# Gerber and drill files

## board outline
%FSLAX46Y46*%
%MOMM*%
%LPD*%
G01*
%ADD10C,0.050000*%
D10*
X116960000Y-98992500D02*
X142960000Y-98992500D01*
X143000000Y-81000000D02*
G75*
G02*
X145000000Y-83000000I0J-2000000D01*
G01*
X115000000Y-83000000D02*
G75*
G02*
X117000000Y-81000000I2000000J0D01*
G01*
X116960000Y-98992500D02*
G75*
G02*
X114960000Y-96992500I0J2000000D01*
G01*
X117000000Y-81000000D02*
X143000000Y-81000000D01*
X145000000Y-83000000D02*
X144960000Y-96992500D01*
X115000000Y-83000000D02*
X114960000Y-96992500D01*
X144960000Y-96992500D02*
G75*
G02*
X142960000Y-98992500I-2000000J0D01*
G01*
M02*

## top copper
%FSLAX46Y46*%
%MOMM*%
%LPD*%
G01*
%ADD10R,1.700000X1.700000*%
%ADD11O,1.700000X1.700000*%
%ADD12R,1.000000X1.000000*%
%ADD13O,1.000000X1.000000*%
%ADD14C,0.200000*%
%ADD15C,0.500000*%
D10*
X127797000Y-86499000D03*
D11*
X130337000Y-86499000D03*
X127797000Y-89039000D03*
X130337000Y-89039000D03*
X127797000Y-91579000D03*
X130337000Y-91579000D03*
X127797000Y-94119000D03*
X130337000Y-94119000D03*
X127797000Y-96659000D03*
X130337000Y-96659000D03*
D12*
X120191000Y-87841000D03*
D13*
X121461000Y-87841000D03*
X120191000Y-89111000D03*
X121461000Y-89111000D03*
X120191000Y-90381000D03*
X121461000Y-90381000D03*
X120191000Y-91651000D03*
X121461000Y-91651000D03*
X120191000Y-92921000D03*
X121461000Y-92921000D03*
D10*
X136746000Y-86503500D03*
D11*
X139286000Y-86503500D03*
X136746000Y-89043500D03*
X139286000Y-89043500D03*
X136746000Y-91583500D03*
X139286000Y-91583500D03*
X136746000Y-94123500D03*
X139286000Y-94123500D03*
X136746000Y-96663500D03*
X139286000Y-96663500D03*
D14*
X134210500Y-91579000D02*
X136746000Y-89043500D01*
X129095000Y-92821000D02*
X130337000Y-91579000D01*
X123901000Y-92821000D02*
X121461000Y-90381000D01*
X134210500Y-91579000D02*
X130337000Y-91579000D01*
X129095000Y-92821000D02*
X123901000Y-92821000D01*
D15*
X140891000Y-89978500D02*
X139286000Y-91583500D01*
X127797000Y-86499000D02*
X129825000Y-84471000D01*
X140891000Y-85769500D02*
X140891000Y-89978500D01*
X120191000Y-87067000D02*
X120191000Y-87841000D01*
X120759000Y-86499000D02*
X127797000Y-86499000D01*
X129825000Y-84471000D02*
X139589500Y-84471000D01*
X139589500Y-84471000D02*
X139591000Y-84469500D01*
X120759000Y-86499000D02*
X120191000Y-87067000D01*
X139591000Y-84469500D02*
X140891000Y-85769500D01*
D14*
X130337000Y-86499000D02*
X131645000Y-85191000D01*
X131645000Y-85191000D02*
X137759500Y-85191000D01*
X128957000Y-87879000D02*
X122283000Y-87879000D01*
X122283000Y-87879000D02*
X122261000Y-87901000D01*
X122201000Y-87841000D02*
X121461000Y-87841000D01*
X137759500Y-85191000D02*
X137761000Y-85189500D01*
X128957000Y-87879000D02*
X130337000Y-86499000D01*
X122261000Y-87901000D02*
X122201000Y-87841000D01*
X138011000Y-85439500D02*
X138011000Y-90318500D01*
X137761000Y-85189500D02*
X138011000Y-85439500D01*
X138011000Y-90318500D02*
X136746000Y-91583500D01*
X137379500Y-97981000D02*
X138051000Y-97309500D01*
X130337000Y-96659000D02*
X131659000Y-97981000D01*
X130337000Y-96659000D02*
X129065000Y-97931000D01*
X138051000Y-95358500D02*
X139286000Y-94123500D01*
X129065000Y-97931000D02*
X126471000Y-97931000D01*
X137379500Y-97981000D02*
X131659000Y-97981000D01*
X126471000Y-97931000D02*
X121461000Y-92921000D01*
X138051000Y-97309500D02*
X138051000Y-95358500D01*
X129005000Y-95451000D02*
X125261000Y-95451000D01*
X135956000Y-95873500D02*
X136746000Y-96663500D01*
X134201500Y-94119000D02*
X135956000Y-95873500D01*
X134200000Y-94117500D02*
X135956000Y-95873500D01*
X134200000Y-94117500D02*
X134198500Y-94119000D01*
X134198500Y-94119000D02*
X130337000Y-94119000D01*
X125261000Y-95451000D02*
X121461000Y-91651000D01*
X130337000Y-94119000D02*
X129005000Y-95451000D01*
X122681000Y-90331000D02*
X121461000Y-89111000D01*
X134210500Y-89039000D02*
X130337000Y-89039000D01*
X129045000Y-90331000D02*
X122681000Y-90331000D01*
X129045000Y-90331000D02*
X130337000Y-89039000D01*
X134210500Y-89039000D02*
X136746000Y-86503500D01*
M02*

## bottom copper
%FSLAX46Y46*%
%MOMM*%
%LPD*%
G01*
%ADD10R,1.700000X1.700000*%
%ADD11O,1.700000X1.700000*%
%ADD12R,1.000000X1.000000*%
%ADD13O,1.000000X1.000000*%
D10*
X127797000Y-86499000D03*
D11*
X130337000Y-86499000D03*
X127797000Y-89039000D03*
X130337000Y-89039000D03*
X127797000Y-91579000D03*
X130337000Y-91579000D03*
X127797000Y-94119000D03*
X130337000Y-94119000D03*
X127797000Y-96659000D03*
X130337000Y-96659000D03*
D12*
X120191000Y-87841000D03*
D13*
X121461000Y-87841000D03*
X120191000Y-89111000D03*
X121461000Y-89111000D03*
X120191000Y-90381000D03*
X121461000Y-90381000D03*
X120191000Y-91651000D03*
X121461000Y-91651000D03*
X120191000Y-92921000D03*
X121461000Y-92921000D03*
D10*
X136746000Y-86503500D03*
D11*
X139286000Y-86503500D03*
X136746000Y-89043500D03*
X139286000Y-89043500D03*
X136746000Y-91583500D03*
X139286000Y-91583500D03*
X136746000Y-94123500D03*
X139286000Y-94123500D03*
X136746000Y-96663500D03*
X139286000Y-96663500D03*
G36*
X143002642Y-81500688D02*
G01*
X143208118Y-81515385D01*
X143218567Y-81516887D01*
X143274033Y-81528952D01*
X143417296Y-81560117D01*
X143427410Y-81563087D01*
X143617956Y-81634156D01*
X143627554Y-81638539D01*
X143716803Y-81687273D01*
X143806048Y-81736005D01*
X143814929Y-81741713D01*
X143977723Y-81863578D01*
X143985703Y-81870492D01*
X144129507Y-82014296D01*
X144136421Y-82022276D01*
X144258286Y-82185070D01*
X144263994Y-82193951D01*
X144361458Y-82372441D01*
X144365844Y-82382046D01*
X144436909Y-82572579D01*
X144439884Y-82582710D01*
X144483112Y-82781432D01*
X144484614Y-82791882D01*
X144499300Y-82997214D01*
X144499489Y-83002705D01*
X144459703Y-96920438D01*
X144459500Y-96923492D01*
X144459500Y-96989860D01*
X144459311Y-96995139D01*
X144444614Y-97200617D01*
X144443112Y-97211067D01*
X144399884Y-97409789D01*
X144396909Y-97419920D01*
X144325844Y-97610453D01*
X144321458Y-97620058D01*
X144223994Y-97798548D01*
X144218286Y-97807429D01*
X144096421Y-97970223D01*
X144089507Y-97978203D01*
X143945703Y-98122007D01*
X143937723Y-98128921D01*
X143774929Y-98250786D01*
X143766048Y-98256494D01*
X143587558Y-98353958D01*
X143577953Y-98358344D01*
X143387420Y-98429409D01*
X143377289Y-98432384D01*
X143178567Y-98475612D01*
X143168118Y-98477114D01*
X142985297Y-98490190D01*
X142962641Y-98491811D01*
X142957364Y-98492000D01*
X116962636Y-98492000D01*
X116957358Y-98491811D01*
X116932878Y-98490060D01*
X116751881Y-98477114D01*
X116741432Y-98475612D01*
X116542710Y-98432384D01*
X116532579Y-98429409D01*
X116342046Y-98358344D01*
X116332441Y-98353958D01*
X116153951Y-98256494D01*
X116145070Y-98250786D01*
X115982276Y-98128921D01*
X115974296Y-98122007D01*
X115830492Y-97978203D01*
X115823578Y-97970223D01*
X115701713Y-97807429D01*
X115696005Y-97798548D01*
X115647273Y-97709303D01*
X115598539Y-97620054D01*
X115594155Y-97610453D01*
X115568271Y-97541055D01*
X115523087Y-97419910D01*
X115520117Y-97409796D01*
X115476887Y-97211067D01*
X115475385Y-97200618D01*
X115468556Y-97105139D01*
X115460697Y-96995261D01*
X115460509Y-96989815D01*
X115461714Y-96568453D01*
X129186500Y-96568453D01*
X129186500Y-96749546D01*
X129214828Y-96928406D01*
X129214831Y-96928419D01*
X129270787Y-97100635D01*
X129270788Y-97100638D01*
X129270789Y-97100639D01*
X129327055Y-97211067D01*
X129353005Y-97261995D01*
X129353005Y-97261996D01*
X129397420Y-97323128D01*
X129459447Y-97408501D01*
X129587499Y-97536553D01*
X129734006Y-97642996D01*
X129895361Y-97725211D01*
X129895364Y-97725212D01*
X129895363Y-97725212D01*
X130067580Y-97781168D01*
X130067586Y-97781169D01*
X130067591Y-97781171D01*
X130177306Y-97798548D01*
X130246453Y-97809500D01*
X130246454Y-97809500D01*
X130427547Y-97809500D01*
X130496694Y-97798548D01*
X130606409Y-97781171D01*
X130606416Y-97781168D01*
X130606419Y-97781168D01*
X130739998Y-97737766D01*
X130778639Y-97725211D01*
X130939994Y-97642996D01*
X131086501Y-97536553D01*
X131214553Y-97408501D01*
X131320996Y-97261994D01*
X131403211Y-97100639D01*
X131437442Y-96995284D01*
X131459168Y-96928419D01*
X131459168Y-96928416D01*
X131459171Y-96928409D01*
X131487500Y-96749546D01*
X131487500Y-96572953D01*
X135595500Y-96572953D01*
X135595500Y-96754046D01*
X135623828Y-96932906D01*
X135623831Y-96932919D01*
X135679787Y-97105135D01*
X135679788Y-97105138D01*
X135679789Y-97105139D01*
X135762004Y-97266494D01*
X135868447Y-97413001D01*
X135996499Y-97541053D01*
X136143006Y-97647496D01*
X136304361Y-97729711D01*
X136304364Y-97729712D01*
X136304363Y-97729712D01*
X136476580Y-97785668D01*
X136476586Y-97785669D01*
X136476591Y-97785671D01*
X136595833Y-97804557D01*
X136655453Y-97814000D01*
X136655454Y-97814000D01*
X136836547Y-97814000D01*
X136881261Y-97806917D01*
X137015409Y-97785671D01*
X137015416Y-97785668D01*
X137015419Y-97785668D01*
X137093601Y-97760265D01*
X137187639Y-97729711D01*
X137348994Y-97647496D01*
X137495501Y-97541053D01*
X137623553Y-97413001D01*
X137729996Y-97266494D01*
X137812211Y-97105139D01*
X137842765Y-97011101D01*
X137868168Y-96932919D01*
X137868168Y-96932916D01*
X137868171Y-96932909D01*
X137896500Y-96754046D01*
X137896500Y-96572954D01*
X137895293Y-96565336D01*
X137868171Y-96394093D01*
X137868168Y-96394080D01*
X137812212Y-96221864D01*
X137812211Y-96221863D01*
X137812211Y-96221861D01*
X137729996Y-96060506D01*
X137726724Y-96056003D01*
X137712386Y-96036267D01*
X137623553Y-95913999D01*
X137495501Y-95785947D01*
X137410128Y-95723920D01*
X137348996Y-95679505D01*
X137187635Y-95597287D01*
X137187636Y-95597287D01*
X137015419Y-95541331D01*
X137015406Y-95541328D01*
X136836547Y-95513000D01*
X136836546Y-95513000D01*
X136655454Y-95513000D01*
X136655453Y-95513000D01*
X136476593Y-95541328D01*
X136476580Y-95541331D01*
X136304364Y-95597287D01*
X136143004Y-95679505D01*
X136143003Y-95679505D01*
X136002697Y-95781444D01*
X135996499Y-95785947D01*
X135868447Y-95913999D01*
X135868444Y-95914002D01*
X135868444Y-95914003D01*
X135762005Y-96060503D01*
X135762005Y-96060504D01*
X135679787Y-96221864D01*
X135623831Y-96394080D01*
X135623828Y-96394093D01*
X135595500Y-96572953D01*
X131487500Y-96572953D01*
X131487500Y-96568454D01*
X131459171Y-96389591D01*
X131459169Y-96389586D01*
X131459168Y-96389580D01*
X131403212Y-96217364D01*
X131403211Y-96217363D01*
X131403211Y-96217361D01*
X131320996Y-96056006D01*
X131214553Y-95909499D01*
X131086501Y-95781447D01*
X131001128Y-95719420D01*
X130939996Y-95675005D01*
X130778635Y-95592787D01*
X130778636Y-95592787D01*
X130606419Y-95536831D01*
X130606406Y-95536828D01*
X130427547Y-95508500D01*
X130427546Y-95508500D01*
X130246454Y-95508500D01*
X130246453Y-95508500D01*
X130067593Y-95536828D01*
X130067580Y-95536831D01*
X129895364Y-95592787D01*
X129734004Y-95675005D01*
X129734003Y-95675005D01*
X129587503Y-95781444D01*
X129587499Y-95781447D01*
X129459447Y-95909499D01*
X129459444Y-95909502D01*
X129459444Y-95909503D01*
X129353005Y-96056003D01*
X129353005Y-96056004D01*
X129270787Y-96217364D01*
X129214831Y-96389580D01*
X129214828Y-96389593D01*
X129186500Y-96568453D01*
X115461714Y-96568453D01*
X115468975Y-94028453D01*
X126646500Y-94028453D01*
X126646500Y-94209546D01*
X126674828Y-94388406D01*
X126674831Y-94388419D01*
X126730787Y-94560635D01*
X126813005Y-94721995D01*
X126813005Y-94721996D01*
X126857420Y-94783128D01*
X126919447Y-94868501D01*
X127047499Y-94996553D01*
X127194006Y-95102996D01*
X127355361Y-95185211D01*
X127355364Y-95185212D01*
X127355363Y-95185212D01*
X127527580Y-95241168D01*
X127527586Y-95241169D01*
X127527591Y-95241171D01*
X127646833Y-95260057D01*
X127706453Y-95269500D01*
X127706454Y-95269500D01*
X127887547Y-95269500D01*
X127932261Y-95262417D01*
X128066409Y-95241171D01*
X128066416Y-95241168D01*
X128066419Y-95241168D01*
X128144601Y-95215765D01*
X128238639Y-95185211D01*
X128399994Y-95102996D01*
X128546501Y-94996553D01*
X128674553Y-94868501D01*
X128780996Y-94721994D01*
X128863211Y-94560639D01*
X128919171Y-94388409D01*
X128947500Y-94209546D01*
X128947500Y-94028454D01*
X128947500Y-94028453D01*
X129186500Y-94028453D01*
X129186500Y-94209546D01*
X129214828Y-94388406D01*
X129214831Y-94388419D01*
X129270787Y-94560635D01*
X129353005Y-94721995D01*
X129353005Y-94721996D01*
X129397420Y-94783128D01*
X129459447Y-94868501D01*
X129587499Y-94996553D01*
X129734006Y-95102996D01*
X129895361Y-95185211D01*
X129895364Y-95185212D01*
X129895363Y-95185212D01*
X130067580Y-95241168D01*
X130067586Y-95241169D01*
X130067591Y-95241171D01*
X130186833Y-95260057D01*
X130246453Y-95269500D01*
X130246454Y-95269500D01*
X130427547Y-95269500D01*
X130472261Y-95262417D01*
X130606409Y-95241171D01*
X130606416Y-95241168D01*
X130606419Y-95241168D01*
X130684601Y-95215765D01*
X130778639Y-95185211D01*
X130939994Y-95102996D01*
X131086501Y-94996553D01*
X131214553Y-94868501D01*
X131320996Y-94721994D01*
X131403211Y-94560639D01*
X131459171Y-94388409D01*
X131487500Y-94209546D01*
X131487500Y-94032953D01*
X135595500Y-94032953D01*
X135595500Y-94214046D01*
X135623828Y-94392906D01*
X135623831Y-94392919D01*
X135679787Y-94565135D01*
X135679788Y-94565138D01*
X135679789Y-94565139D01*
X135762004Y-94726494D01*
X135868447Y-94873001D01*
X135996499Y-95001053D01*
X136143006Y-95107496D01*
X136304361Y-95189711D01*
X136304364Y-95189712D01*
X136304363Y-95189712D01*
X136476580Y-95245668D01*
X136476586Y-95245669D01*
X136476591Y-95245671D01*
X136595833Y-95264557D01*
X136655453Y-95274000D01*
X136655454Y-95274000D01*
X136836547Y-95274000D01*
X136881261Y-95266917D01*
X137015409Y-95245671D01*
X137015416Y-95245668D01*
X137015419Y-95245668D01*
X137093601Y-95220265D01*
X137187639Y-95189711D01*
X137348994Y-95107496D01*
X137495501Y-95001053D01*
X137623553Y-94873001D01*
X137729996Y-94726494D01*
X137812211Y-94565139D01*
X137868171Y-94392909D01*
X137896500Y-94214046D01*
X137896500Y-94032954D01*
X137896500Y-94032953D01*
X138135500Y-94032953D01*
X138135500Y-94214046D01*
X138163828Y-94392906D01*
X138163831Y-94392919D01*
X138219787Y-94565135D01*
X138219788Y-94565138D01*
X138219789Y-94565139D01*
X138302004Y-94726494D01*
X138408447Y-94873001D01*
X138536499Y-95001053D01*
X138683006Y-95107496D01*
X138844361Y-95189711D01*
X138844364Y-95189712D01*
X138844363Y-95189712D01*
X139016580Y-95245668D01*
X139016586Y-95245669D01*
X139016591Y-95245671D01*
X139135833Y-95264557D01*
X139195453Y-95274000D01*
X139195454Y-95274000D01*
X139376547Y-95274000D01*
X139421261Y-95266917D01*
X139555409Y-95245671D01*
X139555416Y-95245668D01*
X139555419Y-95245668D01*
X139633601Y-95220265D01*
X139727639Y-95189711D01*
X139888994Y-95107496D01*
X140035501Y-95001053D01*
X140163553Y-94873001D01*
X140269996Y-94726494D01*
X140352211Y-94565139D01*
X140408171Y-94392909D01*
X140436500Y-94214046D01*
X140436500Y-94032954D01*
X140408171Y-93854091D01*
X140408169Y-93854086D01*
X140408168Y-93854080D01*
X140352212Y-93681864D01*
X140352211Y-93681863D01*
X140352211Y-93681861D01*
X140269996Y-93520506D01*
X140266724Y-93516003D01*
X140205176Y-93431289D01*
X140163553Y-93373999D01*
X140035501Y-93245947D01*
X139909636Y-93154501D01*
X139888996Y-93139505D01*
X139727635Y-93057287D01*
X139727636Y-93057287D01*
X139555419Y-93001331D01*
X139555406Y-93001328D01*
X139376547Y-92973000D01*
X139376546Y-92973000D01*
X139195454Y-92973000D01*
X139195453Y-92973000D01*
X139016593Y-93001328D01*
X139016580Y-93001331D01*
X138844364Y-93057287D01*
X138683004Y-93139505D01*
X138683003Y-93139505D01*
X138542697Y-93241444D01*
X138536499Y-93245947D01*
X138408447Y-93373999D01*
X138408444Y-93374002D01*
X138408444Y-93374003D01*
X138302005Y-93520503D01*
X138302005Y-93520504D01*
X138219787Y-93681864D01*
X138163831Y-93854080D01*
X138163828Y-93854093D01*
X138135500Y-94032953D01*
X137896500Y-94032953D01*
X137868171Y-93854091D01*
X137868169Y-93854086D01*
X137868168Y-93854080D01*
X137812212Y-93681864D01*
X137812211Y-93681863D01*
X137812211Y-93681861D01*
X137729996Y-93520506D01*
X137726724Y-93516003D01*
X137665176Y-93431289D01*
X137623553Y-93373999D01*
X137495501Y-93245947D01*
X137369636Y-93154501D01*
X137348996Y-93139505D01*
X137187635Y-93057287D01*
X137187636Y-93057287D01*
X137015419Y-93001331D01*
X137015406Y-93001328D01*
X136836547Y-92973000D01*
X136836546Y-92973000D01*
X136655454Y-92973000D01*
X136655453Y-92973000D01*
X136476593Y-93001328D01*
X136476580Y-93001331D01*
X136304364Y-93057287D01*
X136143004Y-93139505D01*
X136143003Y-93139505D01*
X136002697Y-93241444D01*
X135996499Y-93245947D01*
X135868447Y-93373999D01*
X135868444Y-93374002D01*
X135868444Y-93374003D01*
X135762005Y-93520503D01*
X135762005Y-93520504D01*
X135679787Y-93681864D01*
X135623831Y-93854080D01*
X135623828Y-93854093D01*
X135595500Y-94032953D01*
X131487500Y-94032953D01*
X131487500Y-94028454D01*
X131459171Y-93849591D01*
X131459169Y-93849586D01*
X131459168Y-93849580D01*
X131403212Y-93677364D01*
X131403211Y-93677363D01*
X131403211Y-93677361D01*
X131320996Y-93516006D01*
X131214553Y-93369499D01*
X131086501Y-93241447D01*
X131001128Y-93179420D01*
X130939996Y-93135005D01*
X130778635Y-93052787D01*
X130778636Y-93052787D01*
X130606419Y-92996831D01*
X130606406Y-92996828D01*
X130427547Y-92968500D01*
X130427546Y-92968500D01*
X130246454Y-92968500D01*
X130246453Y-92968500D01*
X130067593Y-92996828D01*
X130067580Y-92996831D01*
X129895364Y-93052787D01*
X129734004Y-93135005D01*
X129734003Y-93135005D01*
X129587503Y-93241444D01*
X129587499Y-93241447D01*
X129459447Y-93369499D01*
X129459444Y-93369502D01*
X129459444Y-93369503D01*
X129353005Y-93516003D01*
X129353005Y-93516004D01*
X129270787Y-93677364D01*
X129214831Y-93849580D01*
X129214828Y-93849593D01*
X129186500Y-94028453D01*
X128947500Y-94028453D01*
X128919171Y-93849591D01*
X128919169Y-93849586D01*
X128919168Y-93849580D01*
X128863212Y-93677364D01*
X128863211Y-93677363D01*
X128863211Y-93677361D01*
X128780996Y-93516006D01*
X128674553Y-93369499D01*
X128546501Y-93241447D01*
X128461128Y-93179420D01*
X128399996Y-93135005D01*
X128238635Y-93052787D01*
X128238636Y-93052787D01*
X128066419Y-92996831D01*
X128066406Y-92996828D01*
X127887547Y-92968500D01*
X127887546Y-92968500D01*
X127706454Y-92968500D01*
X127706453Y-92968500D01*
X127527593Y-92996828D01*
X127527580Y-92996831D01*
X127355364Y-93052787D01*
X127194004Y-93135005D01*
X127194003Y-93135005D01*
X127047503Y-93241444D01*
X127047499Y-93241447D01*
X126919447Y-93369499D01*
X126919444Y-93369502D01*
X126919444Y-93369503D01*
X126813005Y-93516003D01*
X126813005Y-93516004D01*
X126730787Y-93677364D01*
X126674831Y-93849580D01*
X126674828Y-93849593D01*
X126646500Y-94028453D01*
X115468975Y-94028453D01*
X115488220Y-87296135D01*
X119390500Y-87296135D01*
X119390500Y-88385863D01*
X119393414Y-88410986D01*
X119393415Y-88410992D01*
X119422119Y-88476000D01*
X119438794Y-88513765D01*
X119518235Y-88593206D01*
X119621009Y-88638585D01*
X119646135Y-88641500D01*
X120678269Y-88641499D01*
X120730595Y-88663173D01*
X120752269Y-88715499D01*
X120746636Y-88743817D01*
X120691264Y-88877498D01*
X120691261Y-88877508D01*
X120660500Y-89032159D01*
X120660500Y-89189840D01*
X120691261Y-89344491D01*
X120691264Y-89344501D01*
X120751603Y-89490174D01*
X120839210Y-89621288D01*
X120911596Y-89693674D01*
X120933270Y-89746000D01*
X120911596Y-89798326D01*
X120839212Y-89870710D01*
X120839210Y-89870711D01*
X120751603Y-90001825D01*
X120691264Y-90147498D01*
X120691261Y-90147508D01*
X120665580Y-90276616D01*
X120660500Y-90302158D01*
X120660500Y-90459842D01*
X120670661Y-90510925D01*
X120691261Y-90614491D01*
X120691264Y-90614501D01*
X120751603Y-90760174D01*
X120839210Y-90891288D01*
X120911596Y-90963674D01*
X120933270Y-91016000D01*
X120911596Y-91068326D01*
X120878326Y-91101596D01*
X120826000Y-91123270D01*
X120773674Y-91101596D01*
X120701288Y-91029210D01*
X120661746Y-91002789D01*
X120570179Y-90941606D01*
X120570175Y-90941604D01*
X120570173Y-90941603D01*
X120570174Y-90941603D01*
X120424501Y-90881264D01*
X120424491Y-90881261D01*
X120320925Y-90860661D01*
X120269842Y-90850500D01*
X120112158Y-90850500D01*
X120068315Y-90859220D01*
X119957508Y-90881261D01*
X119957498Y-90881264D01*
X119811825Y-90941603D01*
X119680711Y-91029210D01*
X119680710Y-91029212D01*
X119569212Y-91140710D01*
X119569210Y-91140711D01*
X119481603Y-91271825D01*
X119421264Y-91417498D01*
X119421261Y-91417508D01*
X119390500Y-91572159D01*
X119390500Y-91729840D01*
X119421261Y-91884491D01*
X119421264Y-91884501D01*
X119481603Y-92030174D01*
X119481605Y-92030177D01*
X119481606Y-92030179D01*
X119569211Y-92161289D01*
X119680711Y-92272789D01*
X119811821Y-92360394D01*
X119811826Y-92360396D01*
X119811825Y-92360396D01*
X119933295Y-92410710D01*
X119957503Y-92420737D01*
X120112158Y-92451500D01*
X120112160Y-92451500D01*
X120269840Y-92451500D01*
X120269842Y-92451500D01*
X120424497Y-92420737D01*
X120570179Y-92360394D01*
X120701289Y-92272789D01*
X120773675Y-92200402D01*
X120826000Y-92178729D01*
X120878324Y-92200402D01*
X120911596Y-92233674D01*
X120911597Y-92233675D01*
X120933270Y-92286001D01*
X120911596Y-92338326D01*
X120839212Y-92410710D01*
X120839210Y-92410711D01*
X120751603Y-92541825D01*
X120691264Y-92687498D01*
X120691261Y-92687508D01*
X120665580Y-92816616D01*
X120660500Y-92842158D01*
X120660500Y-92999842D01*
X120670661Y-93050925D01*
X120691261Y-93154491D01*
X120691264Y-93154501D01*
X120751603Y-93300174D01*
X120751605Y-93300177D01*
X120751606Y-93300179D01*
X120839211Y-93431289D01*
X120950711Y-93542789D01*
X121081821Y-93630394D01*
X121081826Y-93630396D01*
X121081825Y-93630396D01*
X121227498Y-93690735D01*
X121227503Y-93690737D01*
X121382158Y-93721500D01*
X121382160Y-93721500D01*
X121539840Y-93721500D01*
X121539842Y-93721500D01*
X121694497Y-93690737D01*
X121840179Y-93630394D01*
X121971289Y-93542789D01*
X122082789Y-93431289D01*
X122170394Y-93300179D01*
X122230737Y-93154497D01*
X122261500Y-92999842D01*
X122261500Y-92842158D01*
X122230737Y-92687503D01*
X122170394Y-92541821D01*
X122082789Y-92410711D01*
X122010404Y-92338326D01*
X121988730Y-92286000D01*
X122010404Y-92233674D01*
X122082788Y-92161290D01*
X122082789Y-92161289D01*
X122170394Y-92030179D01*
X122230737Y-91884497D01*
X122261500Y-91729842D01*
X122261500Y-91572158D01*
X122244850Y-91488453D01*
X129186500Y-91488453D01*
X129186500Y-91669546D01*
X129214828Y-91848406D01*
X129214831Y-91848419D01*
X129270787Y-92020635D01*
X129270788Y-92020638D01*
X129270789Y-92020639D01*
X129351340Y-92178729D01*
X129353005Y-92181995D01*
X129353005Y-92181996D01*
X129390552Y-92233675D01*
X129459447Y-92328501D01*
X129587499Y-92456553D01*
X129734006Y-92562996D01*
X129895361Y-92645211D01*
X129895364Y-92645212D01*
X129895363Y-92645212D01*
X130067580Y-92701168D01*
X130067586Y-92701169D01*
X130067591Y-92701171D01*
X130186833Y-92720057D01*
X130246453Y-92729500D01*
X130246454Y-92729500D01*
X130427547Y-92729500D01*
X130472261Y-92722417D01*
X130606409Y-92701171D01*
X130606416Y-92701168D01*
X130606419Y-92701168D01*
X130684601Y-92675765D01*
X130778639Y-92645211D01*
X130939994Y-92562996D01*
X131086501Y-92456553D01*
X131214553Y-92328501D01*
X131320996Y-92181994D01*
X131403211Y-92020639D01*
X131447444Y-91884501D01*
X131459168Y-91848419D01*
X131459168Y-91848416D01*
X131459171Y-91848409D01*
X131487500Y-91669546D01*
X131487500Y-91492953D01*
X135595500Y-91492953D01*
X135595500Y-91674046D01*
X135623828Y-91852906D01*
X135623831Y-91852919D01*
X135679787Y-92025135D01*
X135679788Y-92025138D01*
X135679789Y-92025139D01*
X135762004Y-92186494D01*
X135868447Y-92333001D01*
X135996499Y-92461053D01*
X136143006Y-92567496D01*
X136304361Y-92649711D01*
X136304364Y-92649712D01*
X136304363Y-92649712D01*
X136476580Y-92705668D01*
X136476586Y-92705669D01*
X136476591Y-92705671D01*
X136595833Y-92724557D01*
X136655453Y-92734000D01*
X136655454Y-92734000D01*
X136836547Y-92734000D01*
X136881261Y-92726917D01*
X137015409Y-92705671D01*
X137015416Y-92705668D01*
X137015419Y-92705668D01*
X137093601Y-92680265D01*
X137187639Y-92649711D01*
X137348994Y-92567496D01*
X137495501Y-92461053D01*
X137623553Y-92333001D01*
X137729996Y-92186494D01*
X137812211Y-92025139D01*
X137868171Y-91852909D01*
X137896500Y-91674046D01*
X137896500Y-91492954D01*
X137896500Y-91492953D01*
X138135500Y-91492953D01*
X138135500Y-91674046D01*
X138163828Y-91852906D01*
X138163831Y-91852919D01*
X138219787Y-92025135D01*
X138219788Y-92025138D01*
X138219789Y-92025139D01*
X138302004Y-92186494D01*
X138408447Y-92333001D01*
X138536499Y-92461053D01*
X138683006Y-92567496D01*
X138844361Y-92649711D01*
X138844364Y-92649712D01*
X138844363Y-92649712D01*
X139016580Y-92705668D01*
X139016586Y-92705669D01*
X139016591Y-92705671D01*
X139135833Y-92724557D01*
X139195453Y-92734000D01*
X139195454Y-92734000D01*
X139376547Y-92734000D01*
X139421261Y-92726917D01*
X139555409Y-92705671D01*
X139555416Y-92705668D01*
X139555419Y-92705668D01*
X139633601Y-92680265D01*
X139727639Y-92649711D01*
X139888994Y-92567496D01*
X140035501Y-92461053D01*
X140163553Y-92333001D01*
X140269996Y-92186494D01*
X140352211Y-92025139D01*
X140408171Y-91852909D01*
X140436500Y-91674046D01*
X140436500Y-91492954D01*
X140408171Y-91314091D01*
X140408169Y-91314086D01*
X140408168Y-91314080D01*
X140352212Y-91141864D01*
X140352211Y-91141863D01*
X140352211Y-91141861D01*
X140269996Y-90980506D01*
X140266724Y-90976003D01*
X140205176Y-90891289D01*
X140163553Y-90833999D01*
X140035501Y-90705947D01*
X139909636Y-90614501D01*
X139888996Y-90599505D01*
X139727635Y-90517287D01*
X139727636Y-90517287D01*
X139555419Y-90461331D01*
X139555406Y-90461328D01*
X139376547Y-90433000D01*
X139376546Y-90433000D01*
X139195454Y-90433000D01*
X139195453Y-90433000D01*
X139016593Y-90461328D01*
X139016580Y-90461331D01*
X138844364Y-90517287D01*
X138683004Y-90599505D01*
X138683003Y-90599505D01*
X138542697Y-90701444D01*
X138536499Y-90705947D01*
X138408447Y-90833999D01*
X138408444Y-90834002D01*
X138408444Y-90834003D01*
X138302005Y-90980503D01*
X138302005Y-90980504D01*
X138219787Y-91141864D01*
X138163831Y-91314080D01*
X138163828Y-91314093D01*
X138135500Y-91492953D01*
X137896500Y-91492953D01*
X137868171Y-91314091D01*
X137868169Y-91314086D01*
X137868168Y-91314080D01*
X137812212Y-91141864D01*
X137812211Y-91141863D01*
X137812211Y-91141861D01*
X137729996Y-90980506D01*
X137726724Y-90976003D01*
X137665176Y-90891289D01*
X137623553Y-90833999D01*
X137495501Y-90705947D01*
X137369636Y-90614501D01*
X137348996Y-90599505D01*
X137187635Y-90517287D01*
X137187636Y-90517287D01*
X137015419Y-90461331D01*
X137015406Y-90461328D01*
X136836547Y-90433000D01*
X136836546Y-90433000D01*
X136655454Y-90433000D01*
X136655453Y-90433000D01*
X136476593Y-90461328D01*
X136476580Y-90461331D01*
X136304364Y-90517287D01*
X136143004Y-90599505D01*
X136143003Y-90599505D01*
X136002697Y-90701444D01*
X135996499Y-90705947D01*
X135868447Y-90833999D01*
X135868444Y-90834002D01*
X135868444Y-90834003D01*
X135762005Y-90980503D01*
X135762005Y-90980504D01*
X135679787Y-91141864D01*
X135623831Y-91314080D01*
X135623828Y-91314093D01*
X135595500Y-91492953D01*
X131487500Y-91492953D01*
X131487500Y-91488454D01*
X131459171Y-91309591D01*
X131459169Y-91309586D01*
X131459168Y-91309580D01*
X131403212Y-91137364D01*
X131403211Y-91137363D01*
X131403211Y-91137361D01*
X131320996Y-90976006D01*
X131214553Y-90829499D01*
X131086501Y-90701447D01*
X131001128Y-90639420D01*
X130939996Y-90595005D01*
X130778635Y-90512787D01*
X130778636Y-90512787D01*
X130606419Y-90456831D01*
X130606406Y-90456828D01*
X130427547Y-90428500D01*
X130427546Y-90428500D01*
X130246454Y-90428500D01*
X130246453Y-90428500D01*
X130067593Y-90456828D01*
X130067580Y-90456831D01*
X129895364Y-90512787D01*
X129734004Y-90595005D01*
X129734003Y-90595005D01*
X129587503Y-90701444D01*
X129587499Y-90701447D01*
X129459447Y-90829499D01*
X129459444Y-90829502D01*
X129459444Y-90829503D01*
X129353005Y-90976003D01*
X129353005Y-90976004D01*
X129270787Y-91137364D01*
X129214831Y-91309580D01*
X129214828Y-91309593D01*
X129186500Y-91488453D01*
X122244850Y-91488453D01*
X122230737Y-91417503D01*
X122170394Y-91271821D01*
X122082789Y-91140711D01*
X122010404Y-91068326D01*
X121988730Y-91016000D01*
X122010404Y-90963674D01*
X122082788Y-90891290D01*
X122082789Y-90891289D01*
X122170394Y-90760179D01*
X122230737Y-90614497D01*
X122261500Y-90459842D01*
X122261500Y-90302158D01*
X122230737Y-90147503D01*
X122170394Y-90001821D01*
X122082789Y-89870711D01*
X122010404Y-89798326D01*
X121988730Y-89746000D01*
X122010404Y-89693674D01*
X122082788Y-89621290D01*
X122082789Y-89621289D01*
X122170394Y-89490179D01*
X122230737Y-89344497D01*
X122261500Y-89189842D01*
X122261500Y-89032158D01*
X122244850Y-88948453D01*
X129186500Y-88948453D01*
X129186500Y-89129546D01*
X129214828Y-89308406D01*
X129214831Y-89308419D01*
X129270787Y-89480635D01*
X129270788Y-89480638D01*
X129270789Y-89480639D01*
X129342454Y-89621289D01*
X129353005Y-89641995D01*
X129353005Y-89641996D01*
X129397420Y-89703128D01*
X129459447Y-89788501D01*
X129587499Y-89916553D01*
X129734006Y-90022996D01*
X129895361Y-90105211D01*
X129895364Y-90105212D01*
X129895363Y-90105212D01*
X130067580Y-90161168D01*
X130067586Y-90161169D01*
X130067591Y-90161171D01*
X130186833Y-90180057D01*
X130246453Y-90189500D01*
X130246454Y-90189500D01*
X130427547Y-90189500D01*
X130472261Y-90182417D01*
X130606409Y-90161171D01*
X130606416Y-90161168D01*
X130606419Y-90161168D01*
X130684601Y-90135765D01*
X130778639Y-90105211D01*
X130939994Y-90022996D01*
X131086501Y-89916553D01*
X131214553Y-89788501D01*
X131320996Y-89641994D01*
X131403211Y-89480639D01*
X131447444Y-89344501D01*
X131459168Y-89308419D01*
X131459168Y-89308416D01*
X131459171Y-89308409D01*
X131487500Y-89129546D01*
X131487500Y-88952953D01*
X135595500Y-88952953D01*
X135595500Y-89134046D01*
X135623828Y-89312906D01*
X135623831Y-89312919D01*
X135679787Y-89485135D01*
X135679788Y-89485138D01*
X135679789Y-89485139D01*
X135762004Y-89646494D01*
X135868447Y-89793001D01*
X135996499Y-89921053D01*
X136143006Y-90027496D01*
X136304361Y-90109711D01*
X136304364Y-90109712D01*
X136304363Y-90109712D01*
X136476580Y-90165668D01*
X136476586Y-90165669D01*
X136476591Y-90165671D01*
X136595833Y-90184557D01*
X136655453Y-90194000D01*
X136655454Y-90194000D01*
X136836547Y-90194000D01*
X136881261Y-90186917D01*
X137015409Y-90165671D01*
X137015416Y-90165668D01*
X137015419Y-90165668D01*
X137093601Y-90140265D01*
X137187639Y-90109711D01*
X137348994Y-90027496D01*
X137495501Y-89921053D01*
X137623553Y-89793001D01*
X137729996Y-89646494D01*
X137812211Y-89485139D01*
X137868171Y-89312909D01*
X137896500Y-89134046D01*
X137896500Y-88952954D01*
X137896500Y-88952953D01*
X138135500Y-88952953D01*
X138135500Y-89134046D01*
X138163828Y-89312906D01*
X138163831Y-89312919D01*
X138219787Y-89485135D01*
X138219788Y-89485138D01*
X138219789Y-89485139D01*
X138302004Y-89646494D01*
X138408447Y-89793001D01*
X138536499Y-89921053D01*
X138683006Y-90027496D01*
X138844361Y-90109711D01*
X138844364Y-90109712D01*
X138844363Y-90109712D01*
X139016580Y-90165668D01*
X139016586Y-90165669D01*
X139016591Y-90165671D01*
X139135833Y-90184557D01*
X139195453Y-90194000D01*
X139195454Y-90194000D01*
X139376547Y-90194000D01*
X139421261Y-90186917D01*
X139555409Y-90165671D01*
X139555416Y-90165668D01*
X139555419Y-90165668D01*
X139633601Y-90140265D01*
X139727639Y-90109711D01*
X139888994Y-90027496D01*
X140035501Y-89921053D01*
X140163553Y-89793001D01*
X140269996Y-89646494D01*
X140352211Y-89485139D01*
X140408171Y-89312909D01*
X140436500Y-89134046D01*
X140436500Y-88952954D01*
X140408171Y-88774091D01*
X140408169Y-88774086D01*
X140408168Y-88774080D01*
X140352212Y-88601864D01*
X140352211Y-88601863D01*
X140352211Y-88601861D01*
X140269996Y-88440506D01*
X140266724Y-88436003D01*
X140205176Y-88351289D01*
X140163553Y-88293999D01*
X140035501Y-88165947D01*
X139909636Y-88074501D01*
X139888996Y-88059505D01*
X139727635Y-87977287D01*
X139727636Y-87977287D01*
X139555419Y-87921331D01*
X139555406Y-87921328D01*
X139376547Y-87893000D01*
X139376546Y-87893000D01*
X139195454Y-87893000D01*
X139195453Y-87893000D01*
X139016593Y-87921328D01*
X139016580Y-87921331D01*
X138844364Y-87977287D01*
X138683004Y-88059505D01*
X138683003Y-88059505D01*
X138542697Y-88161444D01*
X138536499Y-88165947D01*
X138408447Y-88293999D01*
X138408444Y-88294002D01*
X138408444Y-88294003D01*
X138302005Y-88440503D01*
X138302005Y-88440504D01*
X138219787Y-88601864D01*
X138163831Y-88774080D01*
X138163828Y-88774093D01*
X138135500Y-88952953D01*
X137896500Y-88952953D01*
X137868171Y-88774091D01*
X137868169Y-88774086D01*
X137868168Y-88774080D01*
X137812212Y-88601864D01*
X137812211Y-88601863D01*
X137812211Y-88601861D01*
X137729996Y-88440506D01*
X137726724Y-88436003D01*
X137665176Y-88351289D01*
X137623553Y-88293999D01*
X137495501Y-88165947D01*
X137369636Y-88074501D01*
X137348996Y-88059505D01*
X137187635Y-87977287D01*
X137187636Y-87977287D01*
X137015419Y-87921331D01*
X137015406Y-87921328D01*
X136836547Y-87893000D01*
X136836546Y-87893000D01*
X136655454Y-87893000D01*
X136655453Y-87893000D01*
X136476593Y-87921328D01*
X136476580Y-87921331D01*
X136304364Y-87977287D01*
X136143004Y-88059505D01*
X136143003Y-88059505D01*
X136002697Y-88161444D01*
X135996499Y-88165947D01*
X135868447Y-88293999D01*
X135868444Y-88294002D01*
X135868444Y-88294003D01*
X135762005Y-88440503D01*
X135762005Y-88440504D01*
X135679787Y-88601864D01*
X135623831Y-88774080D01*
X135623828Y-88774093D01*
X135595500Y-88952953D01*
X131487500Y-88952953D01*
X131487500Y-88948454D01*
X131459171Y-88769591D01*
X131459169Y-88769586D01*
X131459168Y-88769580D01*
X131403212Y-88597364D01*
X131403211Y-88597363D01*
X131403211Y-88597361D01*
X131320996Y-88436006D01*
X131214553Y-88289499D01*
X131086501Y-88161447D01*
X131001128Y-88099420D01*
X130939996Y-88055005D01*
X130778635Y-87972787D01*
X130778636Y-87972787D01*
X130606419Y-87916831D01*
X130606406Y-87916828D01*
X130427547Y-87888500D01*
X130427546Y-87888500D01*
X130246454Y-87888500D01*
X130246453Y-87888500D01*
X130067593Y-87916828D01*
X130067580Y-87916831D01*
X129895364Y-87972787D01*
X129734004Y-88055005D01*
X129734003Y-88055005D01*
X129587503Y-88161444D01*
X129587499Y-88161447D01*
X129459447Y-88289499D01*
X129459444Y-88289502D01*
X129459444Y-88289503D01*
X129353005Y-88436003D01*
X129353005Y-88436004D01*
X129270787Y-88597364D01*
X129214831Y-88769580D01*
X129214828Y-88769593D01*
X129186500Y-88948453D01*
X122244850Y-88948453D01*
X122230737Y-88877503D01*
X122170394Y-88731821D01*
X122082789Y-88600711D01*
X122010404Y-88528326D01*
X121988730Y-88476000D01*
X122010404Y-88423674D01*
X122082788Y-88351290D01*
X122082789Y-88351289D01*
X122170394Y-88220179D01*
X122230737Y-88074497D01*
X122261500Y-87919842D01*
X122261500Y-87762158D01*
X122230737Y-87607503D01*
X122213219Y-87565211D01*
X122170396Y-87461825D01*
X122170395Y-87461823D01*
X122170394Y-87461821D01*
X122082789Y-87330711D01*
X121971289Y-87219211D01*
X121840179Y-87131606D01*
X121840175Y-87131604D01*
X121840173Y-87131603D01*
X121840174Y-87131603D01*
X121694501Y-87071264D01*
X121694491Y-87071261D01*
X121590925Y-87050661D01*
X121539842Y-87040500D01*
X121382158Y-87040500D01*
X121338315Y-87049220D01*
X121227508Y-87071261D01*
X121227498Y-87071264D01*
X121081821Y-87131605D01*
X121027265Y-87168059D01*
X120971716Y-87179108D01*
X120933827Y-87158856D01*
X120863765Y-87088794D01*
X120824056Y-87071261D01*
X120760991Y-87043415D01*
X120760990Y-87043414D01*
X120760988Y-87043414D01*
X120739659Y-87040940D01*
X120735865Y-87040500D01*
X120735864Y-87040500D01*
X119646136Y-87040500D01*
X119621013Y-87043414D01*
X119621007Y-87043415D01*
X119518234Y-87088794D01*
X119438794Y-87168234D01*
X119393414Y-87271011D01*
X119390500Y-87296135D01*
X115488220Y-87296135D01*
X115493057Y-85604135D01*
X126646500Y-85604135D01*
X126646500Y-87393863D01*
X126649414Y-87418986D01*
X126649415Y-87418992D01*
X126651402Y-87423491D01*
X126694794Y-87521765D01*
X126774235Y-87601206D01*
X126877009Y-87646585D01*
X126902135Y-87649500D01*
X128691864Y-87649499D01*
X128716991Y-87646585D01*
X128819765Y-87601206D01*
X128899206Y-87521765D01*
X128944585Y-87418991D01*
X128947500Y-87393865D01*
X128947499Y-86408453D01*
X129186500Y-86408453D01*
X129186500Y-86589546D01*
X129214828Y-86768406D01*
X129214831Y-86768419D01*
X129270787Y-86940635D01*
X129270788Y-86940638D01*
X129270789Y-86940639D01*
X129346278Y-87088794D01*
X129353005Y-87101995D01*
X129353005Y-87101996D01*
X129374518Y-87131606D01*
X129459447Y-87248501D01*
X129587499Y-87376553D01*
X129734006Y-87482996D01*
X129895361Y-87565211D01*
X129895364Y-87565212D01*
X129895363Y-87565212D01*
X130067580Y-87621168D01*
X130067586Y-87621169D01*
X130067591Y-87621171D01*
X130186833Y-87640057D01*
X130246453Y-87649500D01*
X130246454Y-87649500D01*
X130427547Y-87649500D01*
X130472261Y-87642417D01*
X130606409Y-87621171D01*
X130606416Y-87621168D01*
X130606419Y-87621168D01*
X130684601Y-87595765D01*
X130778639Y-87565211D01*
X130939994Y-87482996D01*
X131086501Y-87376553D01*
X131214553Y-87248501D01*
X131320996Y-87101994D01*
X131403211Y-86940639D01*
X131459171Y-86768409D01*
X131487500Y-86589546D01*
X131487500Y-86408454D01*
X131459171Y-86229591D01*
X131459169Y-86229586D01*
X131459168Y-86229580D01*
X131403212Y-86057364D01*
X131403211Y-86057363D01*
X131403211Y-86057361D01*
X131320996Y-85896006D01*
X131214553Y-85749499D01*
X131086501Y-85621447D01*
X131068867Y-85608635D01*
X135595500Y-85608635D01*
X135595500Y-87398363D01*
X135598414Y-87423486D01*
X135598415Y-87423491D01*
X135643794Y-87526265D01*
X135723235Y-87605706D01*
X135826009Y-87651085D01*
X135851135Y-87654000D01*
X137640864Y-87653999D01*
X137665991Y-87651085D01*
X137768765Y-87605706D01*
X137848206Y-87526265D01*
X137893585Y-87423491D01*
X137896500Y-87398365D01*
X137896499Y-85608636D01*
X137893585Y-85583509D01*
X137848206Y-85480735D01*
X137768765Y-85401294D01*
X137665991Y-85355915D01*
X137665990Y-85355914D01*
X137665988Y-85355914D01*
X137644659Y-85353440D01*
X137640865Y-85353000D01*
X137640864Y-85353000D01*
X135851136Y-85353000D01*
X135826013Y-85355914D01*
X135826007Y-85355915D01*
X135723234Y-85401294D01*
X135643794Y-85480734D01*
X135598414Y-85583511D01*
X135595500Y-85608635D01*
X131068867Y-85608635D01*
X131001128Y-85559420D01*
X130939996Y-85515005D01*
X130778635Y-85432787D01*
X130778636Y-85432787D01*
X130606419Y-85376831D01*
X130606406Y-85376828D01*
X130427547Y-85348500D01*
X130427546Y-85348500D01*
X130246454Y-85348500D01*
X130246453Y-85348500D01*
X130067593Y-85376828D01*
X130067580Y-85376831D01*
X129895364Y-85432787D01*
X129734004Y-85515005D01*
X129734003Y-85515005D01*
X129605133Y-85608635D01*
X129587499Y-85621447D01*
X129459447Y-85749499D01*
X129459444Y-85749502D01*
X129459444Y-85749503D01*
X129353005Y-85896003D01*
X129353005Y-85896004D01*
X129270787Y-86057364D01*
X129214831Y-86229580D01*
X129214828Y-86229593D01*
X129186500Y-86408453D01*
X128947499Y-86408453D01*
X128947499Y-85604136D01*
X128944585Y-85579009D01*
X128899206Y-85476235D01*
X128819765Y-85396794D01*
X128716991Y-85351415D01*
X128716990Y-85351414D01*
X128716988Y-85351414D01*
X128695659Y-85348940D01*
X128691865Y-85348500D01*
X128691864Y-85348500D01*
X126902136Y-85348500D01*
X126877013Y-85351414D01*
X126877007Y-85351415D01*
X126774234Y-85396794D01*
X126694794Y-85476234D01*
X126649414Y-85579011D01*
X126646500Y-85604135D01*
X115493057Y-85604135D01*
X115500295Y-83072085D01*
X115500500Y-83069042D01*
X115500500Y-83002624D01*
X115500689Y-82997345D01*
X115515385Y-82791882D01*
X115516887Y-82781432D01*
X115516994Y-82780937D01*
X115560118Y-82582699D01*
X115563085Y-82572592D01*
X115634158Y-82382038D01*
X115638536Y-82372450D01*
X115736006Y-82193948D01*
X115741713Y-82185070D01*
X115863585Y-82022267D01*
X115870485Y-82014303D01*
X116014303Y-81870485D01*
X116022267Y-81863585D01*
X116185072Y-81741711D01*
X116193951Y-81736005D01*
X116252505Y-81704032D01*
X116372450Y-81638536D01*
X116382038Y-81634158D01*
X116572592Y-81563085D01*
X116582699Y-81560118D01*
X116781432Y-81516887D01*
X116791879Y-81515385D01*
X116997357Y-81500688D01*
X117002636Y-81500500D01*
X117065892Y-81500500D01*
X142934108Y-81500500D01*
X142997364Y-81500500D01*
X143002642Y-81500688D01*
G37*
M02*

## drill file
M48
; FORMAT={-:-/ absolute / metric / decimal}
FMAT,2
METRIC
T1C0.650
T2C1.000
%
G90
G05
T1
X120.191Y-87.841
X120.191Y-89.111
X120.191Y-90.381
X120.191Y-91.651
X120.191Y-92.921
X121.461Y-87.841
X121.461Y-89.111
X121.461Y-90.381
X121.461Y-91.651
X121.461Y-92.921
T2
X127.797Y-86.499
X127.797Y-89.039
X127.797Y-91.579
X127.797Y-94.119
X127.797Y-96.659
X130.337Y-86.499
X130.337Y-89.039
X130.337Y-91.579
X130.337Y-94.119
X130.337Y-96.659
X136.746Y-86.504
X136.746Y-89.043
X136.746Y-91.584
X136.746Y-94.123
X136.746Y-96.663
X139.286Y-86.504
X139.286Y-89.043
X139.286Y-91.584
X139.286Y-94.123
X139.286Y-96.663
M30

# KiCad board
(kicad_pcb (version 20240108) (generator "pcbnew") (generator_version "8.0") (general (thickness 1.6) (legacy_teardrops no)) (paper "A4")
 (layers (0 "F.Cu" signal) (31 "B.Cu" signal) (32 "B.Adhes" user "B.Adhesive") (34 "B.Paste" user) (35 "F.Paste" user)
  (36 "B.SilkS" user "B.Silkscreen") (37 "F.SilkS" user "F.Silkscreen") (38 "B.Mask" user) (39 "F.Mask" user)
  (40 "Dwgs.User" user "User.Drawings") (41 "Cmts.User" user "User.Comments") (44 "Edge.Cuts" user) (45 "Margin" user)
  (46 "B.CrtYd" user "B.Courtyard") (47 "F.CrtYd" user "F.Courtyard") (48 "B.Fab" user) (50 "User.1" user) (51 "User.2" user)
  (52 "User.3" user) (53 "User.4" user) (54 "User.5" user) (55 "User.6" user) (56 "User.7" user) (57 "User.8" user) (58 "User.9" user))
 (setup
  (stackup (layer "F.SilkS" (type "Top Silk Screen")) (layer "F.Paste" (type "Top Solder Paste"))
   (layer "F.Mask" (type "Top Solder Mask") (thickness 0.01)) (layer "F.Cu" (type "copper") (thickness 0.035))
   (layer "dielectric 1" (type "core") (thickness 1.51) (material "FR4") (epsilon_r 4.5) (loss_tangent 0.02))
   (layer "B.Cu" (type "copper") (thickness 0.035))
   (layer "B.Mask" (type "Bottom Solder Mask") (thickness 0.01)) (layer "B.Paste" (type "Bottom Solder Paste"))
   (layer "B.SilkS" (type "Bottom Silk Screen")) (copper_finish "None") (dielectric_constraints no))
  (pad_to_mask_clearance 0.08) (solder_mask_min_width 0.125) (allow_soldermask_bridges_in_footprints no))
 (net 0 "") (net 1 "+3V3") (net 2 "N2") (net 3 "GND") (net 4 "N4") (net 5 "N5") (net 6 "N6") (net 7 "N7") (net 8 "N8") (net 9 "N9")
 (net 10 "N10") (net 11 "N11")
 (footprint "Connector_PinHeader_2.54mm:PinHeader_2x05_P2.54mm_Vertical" (layer "F.Cu") (at 127.797 86.499)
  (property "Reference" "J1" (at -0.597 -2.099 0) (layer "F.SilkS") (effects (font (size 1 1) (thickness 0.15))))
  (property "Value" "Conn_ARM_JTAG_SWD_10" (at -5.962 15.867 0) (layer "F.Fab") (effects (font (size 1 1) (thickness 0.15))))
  (pad "1" thru_hole rect (at 0 0) (size 1.7 1.7) (drill 1) (layers "*.Cu" "*.Mask") (remove_unused_layers no) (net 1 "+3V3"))
  (pad "2" thru_hole oval (at 2.54 0) (size 1.7 1.7) (drill 1) (layers "*.Cu" "*.Mask") (remove_unused_layers no) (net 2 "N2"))
  (pad "3" thru_hole oval (at 0 2.54) (size 1.7 1.7) (drill 1) (layers "*.Cu" "*.Mask") (remove_unused_layers no) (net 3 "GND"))
  (pad "4" thru_hole oval (at 2.54 2.54) (size 1.7 1.7) (drill 1) (layers "*.Cu" "*.Mask") (remove_unused_layers no) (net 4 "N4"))
  (pad "5" thru_hole oval (at 0 5.08) (size 1.7 1.7) (drill 1) (layers "*.Cu" "*.Mask") (remove_unused_layers no) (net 3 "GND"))
  (pad "6" thru_hole oval (at 2.54 5.08) (size 1.7 1.7) (drill 1) (layers "*.Cu" "*.Mask") (remove_unused_layers no) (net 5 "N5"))
  (pad "7" thru_hole oval (at 0 7.62) (size 1.7 1.7) (drill 1) (layers "*.Cu" "*.Mask") (remove_unused_layers no) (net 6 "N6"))
  (pad "8" thru_hole oval (at 2.54 7.62) (size 1.7 1.7) (drill 1) (layers "*.Cu" "*.Mask") (remove_unused_layers no) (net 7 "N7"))
  (pad "9" thru_hole oval (at 0 10.16) (size 1.7 1.7) (drill 1) (layers "*.Cu" "*.Mask") (remove_unused_layers no) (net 3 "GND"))
  (pad "10" thru_hole oval (at 2.54 10.16) (size 1.7 1.7) (drill 1) (layers "*.Cu" "*.Mask") (remove_unused_layers no) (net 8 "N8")))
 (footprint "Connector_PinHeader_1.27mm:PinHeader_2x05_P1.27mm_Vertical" (layer "F.Cu") (at 120.191 87.841)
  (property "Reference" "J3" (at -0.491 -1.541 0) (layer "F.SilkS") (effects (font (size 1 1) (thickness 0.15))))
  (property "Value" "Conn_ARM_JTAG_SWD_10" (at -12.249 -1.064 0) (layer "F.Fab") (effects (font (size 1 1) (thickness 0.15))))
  (pad "1" thru_hole rect (at 0 0) (size 1 1) (drill 0.65) (layers "*.Cu" "*.Mask") (remove_unused_layers no) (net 1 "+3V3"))
  (pad "2" thru_hole oval (at 1.27 0) (size 1 1) (drill 0.65) (layers "*.Cu" "*.Mask") (remove_unused_layers no) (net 2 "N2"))
  (pad "3" thru_hole oval (at 0 1.27) (size 1 1) (drill 0.65) (layers "*.Cu" "*.Mask") (remove_unused_layers no) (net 3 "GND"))
  (pad "4" thru_hole oval (at 1.27 1.27) (size 1 1) (drill 0.65) (layers "*.Cu" "*.Mask") (remove_unused_layers no) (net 4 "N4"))
  (pad "5" thru_hole oval (at 0 2.54) (size 1 1) (drill 0.65) (layers "*.Cu" "*.Mask") (remove_unused_layers no) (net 3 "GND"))
  (pad "6" thru_hole oval (at 1.27 2.54) (size 1 1) (drill 0.65) (layers "*.Cu" "*.Mask") (remove_unused_layers no) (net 5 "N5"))
  (pad "7" thru_hole oval (at 0 3.81) (size 1 1) (drill 0.65) (layers "*.Cu" "*.Mask") (remove_unused_layers no) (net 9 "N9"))
  (pad "8" thru_hole oval (at 1.27 3.81) (size 1 1) (drill 0.65) (layers "*.Cu" "*.Mask") (remove_unused_layers no) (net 7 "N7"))
  (pad "9" thru_hole oval (at 0 5.08) (size 1 1) (drill 0.65) (layers "*.Cu" "*.Mask") (remove_unused_layers no) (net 3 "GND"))
  (pad "10" thru_hole oval (at 1.27 5.08) (size 1 1) (drill 0.65) (layers "*.Cu" "*.Mask") (remove_unused_layers no) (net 8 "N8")))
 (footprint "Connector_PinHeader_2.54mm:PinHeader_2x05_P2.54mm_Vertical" (layer "F.Cu") (at 136.746 86.5035)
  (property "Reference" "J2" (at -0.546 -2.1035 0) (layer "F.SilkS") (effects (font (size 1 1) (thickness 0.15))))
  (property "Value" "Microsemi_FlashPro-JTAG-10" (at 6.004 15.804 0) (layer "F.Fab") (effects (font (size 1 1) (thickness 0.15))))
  (pad "1" thru_hole rect (at 0 0) (size 1.7 1.7) (drill 1) (layers "*.Cu" "*.Mask") (remove_unused_layers no) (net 4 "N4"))
  (pad "2" thru_hole oval (at 2.54 0) (size 1.7 1.7) (drill 1) (layers "*.Cu" "*.Mask") (remove_unused_layers no) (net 3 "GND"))
  (pad "3" thru_hole oval (at 0 2.54) (size 1.7 1.7) (drill 1) (layers "*.Cu" "*.Mask") (remove_unused_layers no) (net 5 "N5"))
  (pad "4" thru_hole oval (at 2.54 2.54) (size 1.7 1.7) (drill 1) (layers "*.Cu" "*.Mask") (remove_unused_layers no) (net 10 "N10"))
  (pad "5" thru_hole oval (at 0 5.08) (size 1.7 1.7) (drill 1) (layers "*.Cu" "*.Mask") (remove_unused_layers no) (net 2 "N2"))
  (pad "6" thru_hole oval (at 2.54 5.08) (size 1.7 1.7) (drill 1) (layers "*.Cu" "*.Mask") (remove_unused_layers no) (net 1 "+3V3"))
  (pad "7" thru_hole oval (at 0 7.62) (size 1.7 1.7) (drill 1) (layers "*.Cu" "*.Mask") (remove_unused_layers no) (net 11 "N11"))
  (pad "8" thru_hole oval (at 2.54 7.62) (size 1.7 1.7) (drill 1) (layers "*.Cu" "*.Mask") (remove_unused_layers no) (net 8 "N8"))
  (pad "9" thru_hole oval (at 0 10.16) (size 1.7 1.7) (drill 1) (layers "*.Cu" "*.Mask") (remove_unused_layers no) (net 7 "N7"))
  (pad "10" thru_hole oval (at 2.54 10.16) (size 1.7 1.7) (drill 1) (layers "*.Cu" "*.Mask") (remove_unused_layers no) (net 3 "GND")))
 (gr_line (start 116.96 98.9925) (end 142.96 98.9925) (stroke (width 0.05) (type default)) (layer "Edge.Cuts"))
 (gr_arc (start 143 81) (mid 144.414214 81.585786) (end 145 83) (stroke (width 0.05) (type default)) (layer "Edge.Cuts"))
 (gr_arc (start 115 83) (mid 115.585786 81.585786) (end 117 81) (stroke (width 0.05) (type default)) (layer "Edge.Cuts"))
 (gr_arc (start 116.96 98.9925) (mid 115.545786 98.406714) (end 114.96 96.9925) (stroke (width 0.05) (type default)) (layer "Edge.Cuts"))
 (gr_line (start 117 81) (end 143 81) (stroke (width 0.05) (type default)) (layer "Edge.Cuts"))
 (gr_line (start 145 83) (end 144.96 96.9925) (stroke (width 0.05) (type default)) (layer "Edge.Cuts"))
 (gr_line (start 115 83) (end 114.96 96.9925) (stroke (width 0.05) (type default)) (layer "Edge.Cuts"))
 (gr_arc (start 144.96 96.9925) (mid 144.374214 98.406714) (end 142.96 98.9925) (stroke (width 0.05) (type default)) (layer "Edge.Cuts"))
 (segment (start 134.2105 91.579) (end 136.746 89.0435) (width 0.2) (layer "F.Cu") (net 5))
 (segment (start 129.095 92.821) (end 130.337 91.579) (width 0.2) (layer "F.Cu") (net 5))
 (segment (start 123.901 92.821) (end 121.461 90.381) (width 0.2) (layer "F.Cu") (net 5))
 (segment (start 134.2105 91.579) (end 130.337 91.579) (width 0.2) (layer "F.Cu") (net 5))
 (segment (start 129.095 92.821) (end 123.901 92.821) (width 0.2) (layer "F.Cu") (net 5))
 (segment (start 140.891 89.9785) (end 139.286 91.5835) (width 0.5) (layer "F.Cu") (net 1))
 (segment (start 127.797 86.499) (end 129.825 84.471) (width 0.5) (layer "F.Cu") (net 1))
 (segment (start 140.891 85.7695) (end 140.891 89.9785) (width 0.5) (layer "F.Cu") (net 1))
 (segment (start 120.191 87.067) (end 120.191 87.841) (width 0.5) (layer "F.Cu") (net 1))
 (segment (start 120.759 86.499) (end 127.797 86.499) (width 0.5) (layer "F.Cu") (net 1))
 (segment (start 129.825 84.471) (end 139.5895 84.471) (width 0.5) (layer "F.Cu") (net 1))
 (segment (start 139.5895 84.471) (end 139.591 84.4695) (width 0.5) (layer "F.Cu") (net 1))
 (segment (start 120.759 86.499) (end 120.191 87.067) (width 0.5) (layer "F.Cu") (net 1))
 (segment (start 139.591 84.4695) (end 140.891 85.7695) (width 0.5) (layer "F.Cu") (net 1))
 (segment (start 130.337 86.499) (end 131.645 85.191) (width 0.2) (layer "F.Cu") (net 2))
 (segment (start 131.645 85.191) (end 137.7595 85.191) (width 0.2) (layer "F.Cu") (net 2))
 (segment (start 128.957 87.879) (end 122.283 87.879) (width 0.2) (layer "F.Cu") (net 2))
 (segment (start 122.283 87.879) (end 122.261 87.901) (width 0.2) (layer "F.Cu") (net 2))
 (segment (start 122.201 87.841) (end 121.461 87.841) (width 0.2) (layer "F.Cu") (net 2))
 (segment (start 137.7595 85.191) (end 137.761 85.1895) (width 0.2) (layer "F.Cu") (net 2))
 (segment (start 128.957 87.879) (end 130.337 86.499) (width 0.2) (layer "F.Cu") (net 2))
 (segment (start 122.261 87.901) (end 122.201 87.841) (width 0.2) (layer "F.Cu") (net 2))
 (segment (start 138.011 85.4395) (end 138.011 90.3185) (width 0.2) (layer "F.Cu") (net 2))
 (segment (start 137.761 85.1895) (end 138.011 85.4395) (width 0.2) (layer "F.Cu") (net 2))
 (segment (start 138.011 90.3185) (end 136.746 91.5835) (width 0.2) (layer "F.Cu") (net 2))
 (segment (start 137.3795 97.981) (end 138.051 97.3095) (width 0.2) (layer "F.Cu") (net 8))
 (segment (start 130.337 96.659) (end 131.659 97.981) (width 0.2) (layer "F.Cu") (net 8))
 (segment (start 130.337 96.659) (end 129.065 97.931) (width 0.2) (layer "F.Cu") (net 8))
 (segment (start 138.051 95.3585) (end 139.286 94.1235) (width 0.2) (layer "F.Cu") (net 8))
 (segment (start 129.065 97.931) (end 126.471 97.931) (width 0.2) (layer "F.Cu") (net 8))
 (segment (start 137.3795 97.981) (end 131.659 97.981) (width 0.2) (layer "F.Cu") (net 8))
 (segment (start 126.471 97.931) (end 121.461 92.921) (width 0.2) (layer "F.Cu") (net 8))
 (segment (start 138.051 97.3095) (end 138.051 95.3585) (width 0.2) (layer "F.Cu") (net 8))
 (segment (start 129.005 95.451) (end 125.261 95.451) (width 0.2) (layer "F.Cu") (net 7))
 (segment (start 135.956 95.8735) (end 136.746 96.6635) (width 0.2) (layer "F.Cu") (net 7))
 (segment (start 134.2015 94.119) (end 135.956 95.8735) (width 0.2) (layer "F.Cu") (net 7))
 (segment (start 134.2 94.1175) (end 135.956 95.8735) (width 0.2) (layer "F.Cu") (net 7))
 (segment (start 134.2 94.1175) (end 134.1985 94.119) (width 0.2) (layer "F.Cu") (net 7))
 (segment (start 134.1985 94.119) (end 130.337 94.119) (width 0.2) (layer "F.Cu") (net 7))
 (segment (start 125.261 95.451) (end 121.461 91.651) (width 0.2) (layer "F.Cu") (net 7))
 (segment (start 130.337 94.119) (end 129.005 95.451) (width 0.2) (layer "F.Cu") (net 7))
 (segment (start 122.681 90.331) (end 121.461 89.111) (width 0.2) (layer "F.Cu") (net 4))
 (segment (start 134.2105 89.039) (end 130.337 89.039) (width 0.2) (layer "F.Cu") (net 4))
 (segment (start 129.045 90.331) (end 122.681 90.331) (width 0.2) (layer "F.Cu") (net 4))
 (segment (start 129.045 90.331) (end 130.337 89.039) (width 0.2) (layer "F.Cu") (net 4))
 (segment (start 134.2105 89.039) (end 136.746 86.5035) (width 0.2) (layer "F.Cu") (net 4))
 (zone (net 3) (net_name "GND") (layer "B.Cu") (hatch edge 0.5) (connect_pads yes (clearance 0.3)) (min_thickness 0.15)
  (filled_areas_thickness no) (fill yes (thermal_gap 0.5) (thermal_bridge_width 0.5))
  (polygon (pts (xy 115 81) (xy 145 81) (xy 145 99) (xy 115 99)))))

